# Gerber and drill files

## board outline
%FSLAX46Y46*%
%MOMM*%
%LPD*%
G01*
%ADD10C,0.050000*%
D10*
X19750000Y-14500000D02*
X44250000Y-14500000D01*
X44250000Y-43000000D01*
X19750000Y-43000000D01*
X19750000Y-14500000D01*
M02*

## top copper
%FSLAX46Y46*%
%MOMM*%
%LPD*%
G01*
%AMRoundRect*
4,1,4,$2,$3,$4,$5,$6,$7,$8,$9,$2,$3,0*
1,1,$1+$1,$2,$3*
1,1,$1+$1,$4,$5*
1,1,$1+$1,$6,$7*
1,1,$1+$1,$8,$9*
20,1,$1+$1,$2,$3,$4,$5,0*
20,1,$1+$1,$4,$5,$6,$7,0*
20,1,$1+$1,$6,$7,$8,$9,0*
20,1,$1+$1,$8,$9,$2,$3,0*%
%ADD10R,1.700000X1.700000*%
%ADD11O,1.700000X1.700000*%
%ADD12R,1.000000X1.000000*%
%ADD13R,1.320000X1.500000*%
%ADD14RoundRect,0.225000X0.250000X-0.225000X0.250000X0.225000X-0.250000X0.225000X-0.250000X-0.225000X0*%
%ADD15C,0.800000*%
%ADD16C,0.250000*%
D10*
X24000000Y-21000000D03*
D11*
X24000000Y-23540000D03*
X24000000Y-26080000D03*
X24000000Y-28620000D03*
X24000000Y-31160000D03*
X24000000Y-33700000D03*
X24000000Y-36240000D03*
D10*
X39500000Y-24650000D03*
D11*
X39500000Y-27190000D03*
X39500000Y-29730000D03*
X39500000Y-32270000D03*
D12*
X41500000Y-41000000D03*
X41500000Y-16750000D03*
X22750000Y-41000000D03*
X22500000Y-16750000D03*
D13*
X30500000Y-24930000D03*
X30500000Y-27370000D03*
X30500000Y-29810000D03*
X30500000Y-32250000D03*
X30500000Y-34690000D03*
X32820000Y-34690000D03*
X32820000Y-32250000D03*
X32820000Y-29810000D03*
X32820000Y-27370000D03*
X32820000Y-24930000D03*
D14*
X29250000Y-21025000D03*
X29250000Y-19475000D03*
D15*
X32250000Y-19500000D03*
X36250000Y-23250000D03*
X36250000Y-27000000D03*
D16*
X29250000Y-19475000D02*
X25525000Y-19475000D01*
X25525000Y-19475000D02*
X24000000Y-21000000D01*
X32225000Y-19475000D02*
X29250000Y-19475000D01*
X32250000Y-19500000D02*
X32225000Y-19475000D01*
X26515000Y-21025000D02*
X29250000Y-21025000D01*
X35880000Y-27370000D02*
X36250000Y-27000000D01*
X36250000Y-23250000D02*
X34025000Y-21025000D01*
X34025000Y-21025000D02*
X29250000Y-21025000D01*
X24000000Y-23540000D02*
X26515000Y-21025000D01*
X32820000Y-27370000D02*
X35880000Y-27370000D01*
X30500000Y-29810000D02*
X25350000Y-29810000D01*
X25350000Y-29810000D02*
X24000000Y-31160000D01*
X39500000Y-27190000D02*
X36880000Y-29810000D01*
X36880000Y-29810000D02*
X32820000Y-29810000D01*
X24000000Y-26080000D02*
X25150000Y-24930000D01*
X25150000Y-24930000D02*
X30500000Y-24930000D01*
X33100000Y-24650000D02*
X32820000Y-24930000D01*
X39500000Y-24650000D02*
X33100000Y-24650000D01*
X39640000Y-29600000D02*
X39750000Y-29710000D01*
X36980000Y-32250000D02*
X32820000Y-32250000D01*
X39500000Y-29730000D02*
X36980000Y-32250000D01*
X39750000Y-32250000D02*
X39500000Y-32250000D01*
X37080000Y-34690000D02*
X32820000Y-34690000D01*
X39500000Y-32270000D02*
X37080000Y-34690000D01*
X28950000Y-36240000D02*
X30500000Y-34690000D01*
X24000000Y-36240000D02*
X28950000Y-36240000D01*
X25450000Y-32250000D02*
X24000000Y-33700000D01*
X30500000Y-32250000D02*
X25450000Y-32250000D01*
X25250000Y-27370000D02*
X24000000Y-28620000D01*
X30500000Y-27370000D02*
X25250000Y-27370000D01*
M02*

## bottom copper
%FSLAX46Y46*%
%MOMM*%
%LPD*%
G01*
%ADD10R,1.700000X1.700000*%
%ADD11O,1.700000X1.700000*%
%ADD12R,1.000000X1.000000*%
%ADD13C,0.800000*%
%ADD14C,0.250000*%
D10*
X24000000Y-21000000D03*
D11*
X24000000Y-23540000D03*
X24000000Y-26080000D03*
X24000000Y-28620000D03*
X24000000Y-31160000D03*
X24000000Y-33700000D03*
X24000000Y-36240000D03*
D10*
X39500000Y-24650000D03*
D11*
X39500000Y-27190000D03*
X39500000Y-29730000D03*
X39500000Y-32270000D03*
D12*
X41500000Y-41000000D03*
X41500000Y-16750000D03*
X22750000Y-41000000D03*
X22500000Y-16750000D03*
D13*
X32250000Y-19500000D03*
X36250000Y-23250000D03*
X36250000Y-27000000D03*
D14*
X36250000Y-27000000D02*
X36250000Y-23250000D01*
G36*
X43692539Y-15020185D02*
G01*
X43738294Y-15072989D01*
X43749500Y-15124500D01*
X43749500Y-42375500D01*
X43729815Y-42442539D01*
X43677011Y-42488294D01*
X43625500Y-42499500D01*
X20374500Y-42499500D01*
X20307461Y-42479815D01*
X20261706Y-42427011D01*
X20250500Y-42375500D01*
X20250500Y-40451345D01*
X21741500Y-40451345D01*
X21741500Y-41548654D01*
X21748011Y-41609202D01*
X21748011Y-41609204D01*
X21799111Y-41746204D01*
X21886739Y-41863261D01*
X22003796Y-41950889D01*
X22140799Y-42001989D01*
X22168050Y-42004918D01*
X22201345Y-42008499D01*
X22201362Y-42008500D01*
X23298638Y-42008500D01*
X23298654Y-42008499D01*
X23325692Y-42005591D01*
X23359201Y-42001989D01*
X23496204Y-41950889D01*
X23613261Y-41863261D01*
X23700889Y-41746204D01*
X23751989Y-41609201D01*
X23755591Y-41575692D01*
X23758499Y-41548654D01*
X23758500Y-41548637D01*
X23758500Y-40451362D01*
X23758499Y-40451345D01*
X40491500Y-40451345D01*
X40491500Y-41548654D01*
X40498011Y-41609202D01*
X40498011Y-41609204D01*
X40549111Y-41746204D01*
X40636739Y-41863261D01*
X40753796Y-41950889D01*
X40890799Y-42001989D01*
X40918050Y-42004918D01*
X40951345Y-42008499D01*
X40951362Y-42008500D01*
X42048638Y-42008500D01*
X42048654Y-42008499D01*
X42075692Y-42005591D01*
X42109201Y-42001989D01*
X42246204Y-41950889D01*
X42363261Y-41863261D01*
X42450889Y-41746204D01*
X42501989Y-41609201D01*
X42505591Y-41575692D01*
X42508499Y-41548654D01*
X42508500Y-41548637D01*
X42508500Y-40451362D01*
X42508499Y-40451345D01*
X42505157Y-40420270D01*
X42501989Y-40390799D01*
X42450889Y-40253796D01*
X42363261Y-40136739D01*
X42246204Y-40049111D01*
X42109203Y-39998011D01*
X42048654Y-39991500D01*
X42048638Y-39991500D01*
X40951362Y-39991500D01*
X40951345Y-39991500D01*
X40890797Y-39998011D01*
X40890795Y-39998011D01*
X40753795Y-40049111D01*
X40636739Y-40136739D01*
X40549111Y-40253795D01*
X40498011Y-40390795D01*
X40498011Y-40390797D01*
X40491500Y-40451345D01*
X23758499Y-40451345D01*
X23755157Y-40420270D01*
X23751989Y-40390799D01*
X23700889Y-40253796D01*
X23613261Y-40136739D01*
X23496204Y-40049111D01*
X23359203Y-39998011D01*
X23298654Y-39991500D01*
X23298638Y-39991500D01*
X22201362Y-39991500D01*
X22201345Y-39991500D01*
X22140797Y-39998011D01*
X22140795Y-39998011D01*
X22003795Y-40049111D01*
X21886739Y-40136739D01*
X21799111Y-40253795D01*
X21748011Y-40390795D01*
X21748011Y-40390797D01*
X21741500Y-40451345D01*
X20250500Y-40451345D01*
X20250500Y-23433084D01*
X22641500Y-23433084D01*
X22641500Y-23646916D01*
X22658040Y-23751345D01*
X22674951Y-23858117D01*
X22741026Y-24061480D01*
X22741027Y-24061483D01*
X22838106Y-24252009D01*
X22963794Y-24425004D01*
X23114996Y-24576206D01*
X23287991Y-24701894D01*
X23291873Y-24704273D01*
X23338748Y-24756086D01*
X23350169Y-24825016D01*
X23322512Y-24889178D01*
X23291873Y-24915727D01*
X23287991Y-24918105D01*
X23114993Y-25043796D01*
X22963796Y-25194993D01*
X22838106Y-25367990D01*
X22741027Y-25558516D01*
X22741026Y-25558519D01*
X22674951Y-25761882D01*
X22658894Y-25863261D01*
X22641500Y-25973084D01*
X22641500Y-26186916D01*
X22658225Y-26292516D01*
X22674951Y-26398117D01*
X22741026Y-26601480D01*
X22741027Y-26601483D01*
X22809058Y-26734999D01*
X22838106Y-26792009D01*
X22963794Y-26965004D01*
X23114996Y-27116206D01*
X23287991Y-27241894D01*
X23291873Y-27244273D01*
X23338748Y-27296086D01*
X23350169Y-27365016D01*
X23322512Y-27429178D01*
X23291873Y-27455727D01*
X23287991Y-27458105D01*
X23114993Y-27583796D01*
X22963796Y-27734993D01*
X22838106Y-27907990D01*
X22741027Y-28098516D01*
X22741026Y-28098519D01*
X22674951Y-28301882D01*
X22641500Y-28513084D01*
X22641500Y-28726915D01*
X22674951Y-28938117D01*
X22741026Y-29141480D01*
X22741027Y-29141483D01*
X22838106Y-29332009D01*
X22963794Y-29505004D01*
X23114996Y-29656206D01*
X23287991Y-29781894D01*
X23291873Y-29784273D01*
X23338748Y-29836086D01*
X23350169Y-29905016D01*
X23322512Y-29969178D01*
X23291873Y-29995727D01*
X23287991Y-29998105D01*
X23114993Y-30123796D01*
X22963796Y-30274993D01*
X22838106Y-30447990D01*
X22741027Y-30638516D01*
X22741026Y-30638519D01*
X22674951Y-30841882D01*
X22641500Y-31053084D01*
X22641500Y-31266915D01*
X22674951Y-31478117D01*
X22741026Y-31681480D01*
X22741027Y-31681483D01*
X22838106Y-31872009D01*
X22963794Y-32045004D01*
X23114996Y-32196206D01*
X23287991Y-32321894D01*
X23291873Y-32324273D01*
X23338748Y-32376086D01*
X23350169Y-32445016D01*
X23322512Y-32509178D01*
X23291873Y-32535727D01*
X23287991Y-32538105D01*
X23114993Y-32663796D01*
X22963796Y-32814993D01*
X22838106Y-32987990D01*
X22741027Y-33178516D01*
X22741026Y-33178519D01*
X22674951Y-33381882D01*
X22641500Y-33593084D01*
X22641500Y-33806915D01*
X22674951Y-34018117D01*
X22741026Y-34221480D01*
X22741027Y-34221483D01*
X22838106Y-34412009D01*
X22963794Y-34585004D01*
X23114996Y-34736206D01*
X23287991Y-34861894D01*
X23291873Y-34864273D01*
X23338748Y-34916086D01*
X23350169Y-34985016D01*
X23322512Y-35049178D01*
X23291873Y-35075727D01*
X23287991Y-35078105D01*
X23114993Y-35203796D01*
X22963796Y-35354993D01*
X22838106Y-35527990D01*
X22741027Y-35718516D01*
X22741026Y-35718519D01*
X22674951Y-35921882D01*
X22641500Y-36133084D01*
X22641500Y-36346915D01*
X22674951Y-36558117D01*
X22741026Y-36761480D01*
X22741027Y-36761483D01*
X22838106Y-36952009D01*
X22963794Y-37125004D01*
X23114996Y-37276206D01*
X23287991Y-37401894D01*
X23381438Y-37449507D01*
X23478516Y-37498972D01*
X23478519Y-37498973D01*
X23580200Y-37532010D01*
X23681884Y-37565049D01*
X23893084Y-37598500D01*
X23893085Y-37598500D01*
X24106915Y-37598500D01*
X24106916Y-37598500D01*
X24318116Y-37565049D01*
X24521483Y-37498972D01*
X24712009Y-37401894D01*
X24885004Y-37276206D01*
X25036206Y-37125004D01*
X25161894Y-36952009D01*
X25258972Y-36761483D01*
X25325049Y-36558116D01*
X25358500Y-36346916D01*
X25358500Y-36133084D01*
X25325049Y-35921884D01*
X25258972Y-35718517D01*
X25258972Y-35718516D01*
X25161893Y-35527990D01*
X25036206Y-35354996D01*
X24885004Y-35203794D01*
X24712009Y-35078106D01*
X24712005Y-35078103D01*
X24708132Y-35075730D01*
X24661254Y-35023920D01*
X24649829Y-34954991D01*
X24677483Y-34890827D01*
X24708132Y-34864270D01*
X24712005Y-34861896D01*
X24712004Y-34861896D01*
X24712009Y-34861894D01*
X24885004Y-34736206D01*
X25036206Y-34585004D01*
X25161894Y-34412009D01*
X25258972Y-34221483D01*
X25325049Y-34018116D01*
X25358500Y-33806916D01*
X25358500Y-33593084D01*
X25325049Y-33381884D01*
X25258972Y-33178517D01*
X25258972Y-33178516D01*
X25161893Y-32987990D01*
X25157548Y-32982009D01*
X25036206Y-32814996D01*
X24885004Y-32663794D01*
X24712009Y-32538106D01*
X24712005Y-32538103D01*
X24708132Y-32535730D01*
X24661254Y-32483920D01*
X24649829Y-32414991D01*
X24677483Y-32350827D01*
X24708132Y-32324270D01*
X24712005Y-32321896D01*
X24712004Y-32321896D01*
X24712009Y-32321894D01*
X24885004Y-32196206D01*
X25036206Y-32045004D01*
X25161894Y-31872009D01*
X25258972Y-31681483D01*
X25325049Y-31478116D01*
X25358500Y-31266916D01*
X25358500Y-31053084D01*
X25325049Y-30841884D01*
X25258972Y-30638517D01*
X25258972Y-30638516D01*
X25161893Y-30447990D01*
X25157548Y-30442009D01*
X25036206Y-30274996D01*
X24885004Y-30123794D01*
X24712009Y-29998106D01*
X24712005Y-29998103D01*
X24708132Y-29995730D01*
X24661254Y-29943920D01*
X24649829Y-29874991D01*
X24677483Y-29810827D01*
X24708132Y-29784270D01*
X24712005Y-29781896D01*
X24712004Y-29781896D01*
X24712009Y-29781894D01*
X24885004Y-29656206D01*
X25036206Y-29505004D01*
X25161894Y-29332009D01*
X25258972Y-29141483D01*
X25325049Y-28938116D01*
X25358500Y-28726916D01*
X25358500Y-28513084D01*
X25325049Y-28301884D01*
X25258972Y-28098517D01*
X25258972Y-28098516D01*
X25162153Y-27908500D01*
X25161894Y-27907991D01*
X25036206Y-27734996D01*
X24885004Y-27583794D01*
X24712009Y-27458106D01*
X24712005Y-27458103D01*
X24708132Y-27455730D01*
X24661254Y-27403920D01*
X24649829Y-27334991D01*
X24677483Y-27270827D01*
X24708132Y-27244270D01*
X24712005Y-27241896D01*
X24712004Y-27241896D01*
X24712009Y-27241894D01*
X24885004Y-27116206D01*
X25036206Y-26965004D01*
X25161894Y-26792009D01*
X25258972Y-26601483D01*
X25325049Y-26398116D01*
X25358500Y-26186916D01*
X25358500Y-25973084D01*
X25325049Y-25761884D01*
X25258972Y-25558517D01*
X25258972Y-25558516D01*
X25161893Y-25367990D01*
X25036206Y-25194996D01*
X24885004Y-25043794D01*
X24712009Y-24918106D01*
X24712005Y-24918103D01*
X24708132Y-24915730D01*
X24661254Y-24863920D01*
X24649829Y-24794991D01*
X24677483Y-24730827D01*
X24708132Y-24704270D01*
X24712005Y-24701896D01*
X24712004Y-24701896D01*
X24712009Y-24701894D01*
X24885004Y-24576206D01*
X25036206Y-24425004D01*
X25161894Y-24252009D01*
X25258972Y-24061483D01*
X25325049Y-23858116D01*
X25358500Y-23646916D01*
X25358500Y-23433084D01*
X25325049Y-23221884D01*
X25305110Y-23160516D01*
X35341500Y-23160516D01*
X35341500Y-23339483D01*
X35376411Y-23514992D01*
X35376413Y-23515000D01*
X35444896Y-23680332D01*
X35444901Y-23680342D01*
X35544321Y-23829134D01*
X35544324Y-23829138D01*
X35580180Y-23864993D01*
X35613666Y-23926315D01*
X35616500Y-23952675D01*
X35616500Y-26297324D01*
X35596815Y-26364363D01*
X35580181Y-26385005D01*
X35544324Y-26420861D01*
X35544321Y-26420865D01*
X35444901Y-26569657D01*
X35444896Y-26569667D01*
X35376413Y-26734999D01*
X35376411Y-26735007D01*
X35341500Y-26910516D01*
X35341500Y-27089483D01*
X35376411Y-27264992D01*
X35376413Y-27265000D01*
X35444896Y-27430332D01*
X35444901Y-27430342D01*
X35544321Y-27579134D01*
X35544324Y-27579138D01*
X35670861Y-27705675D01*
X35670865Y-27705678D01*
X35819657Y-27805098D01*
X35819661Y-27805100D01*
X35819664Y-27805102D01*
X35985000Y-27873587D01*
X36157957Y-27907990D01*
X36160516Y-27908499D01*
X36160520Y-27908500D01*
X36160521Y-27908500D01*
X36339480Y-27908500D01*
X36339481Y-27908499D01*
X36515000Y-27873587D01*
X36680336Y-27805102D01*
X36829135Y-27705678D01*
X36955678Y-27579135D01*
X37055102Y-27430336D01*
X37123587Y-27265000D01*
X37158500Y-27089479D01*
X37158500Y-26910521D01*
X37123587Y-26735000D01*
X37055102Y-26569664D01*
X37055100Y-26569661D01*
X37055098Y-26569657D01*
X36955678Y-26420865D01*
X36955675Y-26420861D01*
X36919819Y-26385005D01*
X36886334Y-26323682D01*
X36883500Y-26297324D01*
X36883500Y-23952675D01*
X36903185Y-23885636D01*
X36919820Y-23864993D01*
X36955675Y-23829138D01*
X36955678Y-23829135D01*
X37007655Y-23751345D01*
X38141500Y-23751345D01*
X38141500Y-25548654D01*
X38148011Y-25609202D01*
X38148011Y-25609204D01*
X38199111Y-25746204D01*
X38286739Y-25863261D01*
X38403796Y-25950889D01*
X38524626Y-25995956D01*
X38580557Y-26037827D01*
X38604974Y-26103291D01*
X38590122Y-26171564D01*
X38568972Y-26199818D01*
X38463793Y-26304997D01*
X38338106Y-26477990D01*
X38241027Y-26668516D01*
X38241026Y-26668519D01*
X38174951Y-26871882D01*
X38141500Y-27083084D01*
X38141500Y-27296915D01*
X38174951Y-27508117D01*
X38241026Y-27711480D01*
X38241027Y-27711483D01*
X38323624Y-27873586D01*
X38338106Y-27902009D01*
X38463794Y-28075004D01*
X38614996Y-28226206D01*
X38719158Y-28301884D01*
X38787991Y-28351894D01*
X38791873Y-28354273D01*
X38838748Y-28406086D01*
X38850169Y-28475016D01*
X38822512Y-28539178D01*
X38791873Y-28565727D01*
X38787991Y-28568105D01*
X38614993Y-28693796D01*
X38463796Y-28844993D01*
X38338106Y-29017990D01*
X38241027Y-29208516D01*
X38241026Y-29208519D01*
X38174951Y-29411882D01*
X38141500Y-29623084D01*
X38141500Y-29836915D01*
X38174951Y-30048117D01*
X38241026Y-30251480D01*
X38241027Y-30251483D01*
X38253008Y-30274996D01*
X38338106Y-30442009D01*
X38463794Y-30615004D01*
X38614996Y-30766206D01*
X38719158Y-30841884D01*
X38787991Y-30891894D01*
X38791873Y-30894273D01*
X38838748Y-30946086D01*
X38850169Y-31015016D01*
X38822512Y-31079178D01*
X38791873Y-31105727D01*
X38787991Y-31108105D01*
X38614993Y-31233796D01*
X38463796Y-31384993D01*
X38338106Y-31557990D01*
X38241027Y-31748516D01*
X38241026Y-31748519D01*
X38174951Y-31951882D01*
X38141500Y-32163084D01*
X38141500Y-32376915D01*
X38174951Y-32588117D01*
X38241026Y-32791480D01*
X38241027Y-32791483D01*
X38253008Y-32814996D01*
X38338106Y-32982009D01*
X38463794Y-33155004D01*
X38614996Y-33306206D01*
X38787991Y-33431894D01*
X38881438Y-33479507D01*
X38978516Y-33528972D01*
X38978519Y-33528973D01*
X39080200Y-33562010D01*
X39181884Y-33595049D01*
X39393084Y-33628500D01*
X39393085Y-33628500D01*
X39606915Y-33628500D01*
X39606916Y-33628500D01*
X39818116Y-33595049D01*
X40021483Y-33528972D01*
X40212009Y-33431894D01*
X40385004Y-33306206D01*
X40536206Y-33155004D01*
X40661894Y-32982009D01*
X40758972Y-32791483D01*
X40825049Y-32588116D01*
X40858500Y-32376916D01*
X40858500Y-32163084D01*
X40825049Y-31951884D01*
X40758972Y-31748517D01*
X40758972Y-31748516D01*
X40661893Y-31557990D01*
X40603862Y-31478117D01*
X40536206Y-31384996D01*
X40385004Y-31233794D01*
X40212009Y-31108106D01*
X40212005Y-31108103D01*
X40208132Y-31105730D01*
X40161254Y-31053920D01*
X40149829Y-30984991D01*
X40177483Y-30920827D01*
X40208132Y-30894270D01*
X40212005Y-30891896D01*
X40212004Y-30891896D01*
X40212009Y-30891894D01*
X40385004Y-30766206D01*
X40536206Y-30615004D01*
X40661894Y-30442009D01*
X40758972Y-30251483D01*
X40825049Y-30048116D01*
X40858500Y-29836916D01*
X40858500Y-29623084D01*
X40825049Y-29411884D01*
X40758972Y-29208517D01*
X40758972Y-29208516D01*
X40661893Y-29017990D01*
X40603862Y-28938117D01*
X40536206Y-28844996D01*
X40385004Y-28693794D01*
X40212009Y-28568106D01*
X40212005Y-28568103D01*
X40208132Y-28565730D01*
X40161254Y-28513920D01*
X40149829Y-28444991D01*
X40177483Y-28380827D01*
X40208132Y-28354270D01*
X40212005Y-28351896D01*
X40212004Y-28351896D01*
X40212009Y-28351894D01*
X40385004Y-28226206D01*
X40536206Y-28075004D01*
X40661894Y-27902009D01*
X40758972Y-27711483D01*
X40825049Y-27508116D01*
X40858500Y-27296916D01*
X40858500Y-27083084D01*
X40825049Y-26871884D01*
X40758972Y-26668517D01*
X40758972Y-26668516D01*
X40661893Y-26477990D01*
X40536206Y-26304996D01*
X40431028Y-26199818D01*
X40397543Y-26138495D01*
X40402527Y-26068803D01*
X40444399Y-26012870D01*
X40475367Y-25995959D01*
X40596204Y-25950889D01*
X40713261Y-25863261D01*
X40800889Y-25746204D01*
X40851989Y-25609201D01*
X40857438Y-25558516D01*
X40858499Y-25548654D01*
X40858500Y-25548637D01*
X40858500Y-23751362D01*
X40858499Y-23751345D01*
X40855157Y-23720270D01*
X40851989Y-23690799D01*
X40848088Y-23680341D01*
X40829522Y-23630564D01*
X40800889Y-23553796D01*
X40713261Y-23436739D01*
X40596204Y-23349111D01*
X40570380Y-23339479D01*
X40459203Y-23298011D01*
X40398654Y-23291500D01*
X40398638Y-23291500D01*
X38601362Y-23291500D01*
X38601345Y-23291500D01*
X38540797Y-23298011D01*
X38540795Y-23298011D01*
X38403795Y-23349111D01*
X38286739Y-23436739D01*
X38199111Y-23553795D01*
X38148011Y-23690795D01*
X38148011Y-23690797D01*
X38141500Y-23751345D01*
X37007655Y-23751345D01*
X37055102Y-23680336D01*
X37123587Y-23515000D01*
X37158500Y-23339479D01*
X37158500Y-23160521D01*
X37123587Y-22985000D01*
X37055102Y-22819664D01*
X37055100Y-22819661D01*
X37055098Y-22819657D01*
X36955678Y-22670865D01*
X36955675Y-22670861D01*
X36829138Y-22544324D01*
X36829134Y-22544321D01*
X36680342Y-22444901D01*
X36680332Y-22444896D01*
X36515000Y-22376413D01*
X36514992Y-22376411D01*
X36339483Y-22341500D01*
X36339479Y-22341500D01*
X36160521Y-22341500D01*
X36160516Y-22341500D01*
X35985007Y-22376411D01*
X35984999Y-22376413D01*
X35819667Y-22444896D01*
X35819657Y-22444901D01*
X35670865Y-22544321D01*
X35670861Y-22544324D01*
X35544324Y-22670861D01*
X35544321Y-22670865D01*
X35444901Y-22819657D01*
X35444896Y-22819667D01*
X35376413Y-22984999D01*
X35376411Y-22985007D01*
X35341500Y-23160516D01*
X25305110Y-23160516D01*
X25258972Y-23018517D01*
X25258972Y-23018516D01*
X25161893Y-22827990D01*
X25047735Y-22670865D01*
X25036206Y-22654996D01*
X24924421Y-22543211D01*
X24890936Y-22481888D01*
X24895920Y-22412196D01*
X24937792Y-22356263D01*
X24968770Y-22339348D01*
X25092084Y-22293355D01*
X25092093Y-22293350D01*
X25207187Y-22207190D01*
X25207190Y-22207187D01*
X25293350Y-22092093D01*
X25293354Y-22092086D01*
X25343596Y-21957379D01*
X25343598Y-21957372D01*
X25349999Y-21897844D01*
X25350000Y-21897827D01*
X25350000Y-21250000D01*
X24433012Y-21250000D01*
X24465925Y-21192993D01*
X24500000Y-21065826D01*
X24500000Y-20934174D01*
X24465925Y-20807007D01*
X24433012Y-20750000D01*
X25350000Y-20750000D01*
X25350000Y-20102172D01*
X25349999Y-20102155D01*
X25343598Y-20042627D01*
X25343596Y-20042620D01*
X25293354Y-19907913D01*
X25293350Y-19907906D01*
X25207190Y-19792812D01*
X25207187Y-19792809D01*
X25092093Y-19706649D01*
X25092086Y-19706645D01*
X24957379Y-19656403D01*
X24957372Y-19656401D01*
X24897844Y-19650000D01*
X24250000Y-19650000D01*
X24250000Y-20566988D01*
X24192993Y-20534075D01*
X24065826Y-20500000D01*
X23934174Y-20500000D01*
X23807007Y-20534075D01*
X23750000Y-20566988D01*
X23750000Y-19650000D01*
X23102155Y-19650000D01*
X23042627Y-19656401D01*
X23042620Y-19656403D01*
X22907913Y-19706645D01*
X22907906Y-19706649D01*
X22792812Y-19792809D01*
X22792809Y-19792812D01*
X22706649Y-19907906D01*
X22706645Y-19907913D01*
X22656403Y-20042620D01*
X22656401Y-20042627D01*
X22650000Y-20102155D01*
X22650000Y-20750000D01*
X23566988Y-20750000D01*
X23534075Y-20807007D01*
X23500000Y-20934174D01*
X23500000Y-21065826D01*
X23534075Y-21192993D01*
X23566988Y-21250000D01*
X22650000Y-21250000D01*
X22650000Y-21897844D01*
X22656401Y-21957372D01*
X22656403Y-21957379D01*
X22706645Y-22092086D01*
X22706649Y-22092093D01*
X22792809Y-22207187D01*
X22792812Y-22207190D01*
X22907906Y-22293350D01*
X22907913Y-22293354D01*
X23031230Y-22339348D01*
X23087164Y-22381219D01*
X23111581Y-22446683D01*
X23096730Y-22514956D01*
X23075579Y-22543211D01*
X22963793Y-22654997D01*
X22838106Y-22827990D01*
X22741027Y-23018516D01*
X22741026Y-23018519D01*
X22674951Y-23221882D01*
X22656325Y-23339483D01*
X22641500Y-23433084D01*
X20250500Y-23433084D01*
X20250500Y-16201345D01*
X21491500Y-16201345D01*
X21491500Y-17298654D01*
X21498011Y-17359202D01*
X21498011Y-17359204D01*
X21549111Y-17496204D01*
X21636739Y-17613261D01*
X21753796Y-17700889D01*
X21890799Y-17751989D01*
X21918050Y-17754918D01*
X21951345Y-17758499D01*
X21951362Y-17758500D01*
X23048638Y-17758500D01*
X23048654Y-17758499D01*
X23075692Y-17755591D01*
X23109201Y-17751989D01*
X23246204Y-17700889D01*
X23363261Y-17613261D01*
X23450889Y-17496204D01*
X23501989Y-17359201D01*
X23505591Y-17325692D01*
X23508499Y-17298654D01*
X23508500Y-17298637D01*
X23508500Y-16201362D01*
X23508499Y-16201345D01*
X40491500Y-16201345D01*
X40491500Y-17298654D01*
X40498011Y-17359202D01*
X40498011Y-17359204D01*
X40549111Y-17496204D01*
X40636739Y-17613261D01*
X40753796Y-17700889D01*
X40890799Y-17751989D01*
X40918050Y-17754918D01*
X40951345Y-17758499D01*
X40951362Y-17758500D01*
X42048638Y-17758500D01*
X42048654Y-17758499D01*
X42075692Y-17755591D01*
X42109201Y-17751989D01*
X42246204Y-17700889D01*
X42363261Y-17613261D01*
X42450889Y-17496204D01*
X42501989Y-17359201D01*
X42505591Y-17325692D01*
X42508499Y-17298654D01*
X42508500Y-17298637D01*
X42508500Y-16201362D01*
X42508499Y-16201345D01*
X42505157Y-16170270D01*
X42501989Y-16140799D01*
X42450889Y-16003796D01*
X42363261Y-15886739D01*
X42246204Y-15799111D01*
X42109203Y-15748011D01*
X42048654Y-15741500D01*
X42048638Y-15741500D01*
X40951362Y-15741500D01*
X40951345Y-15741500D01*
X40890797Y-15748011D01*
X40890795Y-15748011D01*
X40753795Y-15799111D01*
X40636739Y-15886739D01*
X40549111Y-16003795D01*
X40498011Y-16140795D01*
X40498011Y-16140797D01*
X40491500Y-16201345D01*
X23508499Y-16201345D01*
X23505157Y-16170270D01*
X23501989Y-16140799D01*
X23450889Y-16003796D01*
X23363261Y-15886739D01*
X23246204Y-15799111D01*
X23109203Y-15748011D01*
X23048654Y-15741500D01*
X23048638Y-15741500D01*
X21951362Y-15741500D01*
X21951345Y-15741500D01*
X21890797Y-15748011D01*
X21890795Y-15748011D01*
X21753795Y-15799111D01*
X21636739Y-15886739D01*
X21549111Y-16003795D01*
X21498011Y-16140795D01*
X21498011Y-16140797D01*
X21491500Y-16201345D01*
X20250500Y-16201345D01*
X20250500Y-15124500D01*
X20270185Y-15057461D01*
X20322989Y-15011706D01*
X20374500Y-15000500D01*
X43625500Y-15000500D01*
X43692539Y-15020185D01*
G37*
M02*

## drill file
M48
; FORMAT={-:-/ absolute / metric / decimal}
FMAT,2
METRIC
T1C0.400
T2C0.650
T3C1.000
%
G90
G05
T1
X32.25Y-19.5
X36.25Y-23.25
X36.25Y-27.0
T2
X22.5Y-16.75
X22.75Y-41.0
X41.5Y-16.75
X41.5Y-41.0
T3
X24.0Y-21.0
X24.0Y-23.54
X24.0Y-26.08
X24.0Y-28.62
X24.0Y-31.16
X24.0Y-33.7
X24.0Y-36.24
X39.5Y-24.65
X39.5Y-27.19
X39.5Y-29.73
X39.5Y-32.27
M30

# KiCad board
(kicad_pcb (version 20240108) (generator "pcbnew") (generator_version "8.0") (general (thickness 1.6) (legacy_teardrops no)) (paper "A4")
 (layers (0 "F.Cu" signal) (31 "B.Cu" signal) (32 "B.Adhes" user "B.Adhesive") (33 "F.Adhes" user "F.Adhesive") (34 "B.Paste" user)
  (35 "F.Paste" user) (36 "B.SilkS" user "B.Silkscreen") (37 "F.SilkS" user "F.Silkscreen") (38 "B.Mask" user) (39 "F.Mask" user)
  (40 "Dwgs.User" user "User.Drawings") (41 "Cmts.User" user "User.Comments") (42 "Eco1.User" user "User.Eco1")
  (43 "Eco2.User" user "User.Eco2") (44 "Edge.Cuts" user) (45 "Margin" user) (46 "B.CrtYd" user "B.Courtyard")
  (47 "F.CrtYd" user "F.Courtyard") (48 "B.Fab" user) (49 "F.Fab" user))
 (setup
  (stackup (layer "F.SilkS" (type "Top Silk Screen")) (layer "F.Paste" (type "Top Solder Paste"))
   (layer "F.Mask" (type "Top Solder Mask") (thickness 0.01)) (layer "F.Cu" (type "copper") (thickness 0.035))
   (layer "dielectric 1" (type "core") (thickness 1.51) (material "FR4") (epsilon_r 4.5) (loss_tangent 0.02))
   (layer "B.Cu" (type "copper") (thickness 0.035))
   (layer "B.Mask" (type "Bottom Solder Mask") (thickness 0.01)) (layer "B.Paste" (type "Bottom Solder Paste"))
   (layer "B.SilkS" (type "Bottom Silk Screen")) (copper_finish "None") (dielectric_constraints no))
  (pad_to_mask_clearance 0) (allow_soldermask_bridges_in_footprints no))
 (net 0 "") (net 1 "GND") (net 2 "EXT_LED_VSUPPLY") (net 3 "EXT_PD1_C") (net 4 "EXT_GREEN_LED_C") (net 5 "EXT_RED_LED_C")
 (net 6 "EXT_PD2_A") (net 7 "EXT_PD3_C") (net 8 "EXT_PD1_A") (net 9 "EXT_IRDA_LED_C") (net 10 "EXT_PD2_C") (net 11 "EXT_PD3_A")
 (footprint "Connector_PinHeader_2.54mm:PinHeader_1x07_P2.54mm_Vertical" (layer "F.Cu") (at 24 21)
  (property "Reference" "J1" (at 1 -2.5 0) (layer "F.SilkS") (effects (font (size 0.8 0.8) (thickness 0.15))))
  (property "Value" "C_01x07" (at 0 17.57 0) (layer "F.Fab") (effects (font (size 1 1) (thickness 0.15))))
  (pad "1" thru_hole rect (at 0 0) (size 1.7 1.7) (drill 1) (layers "*.Cu" "*.Mask") (remove_unused_layers no) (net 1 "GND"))
  (pad "2" thru_hole oval (at 0 2.54) (size 1.7 1.7) (drill 1) (layers "*.Cu" "*.Mask") (remove_unused_layers no) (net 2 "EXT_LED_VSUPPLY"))
  (pad "3" thru_hole oval (at 0 5.08) (size 1.7 1.7) (drill 1) (layers "*.Cu" "*.Mask") (remove_unused_layers no) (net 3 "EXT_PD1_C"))
  (pad "4" thru_hole oval (at 0 7.62) (size 1.7 1.7) (drill 1) (layers "*.Cu" "*.Mask") (remove_unused_layers no) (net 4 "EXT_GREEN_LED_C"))
  (pad "5" thru_hole oval (at 0 10.16) (size 1.7 1.7) (drill 1) (layers "*.Cu" "*.Mask") (remove_unused_layers no) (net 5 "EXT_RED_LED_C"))
  (pad "6" thru_hole oval (at 0 12.7) (size 1.7 1.7) (drill 1) (layers "*.Cu" "*.Mask") (remove_unused_layers no) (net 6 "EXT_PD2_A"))
  (pad "7" thru_hole oval (at 0 15.24) (size 1.7 1.7) (drill 1) (layers "*.Cu" "*.Mask") (remove_unused_layers no) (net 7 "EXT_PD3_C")))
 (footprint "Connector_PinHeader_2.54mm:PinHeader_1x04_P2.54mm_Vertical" (layer "F.Cu") (at 39.5 24.65)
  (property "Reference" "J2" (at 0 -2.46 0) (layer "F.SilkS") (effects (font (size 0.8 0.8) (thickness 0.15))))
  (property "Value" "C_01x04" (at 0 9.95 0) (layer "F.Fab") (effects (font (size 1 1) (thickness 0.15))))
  (pad "1" thru_hole rect (at 0 0) (size 1.7 1.7) (drill 1) (layers "*.Cu" "*.Mask") (remove_unused_layers no) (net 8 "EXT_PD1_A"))
  (pad "2" thru_hole oval (at 0 2.54) (size 1.7 1.7) (drill 1) (layers "*.Cu" "*.Mask") (remove_unused_layers no) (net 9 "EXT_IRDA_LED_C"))
  (pad "3" thru_hole oval (at 0 5.08) (size 1.7 1.7) (drill 1) (layers "*.Cu" "*.Mask") (remove_unused_layers no) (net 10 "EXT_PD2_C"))
  (pad "4" thru_hole oval (at 0 7.62) (size 1.7 1.7) (drill 1) (layers "*.Cu" "*.Mask") (remove_unused_layers no) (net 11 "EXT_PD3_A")))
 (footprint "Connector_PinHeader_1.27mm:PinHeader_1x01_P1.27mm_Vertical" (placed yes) (layer "F.Cu") (at 41.5 41 180)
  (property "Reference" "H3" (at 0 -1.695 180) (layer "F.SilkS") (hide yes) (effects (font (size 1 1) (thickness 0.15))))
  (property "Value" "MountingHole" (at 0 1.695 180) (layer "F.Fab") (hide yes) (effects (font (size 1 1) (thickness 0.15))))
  (pad "1" thru_hole rect (at 0 0 180) (size 1 1) (drill 0.65) (layers "*.Cu" "*.Mask") (remove_unused_layers no)))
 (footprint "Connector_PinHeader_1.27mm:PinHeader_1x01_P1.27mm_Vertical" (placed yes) (layer "F.Cu") (at 41.5 16.75)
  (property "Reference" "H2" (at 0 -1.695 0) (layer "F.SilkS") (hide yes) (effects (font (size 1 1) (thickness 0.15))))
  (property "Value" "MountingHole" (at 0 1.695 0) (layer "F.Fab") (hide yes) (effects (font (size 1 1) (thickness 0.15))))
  (pad "1" thru_hole rect (at 0 0) (size 1 1) (drill 0.65) (layers "*.Cu" "*.Mask") (remove_unused_layers no)))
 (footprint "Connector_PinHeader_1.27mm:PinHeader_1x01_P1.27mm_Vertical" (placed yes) (layer "F.Cu") (at 22.75 41 180)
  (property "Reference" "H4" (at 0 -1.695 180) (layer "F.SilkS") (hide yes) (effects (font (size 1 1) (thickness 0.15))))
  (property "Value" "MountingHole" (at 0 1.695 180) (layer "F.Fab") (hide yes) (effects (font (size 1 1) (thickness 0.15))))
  (pad "1" thru_hole rect (at 0 0 180) (size 1 1) (drill 0.65) (layers "*.Cu" "*.Mask") (remove_unused_layers no)))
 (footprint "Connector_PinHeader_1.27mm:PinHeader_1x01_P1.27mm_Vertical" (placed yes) (layer "F.Cu") (at 22.5 16.75)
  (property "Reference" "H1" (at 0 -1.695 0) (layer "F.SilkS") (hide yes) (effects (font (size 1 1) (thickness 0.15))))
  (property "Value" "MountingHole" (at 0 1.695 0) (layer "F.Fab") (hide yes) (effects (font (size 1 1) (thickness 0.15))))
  (pad "1" thru_hole rect (at 0 0) (size 1 1) (drill 0.65) (layers "*.Cu" "*.Mask") (remove_unused_layers no)))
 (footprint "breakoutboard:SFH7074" (layer "F.Cu") (at 31.66 29.81 -90)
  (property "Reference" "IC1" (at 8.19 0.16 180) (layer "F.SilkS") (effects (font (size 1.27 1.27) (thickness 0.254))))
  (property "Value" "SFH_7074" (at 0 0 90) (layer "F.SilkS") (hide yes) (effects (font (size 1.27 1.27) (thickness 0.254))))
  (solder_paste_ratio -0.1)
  (pad "1" smd rect (at -4.88 1.16) (size 1.32 1.5) (layers "F.Cu" "F.Paste" "F.Mask") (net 3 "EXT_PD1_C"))
  (pad "2" smd rect (at -2.44 1.16) (size 1.32 1.5) (layers "F.Cu" "F.Paste" "F.Mask") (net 4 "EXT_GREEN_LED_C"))
  (pad "3" smd rect (at 0 1.16) (size 1.32 1.5) (layers "F.Cu" "F.Paste" "F.Mask") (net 5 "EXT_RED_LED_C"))
  (pad "4" smd rect (at 2.44 1.16) (size 1.32 1.5) (layers "F.Cu" "F.Paste" "F.Mask") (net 6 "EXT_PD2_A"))
  (pad "5" smd rect (at 4.88 1.16) (size 1.32 1.5) (layers "F.Cu" "F.Paste" "F.Mask") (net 7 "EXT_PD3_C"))
  (pad "6" smd rect (at 4.88 -1.16) (size 1.32 1.5) (layers "F.Cu" "F.Paste" "F.Mask") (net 11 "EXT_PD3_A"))
  (pad "7" smd rect (at 2.44 -1.16) (size 1.32 1.5) (layers "F.Cu" "F.Paste" "F.Mask") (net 10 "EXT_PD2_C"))
  (pad "8" smd rect (at 0 -1.16) (size 1.32 1.5) (layers "F.Cu" "F.Paste" "F.Mask") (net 9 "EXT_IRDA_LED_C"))
  (pad "9" smd rect (at -2.44 -1.16) (size 1.32 1.5) (layers "F.Cu" "F.Paste" "F.Mask") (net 2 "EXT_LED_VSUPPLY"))
  (pad "10" smd rect (at -4.88 -1.16) (size 1.32 1.5) (layers "F.Cu" "F.Paste" "F.Mask") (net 8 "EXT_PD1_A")))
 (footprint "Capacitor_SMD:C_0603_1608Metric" (layer "F.Cu") (at 29.25 20.25 90)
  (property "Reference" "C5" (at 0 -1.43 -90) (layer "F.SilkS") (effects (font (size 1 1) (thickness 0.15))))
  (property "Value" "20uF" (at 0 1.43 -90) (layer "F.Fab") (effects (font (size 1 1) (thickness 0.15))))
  (pad "1" smd roundrect (at -0.775 0 90) (size 0.9 0.95) (layers "F.Cu" "F.Paste" "F.Mask") (roundrect_rratio 0.25)
   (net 2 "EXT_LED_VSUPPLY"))
  (pad "2" smd roundrect (at 0.775 0 90) (size 0.9 0.95) (layers "F.Cu" "F.Paste" "F.Mask") (roundrect_rratio 0.25) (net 1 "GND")))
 (gr_rect (start 19.75 14.5) (end 44.25 43) (stroke (width 0.05) (type solid)) (fill none) (layer "Edge.Cuts"))
 (segment (start 29.25 19.475) (end 25.525 19.475) (width 0.25) (layer "F.Cu") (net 1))
 (segment (start 25.525 19.475) (end 24 21) (width 0.25) (layer "F.Cu") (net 1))
 (segment (start 32.225 19.475) (end 29.25 19.475) (width 0.25) (layer "F.Cu") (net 1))
 (segment (start 32.25 19.5) (end 32.225 19.475) (width 0.25) (layer "F.Cu") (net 1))
 (via (at 32.25 19.5) (size 0.8) (drill 0.4) (layers "F.Cu" "B.Cu") (free yes) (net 1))
 (segment (start 26.515 21.025) (end 29.25 21.025) (width 0.25) (layer "F.Cu") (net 2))
 (segment (start 35.88 27.37) (end 36.25 27) (width 0.25) (layer "F.Cu") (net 2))
 (segment (start 36.25 23.25) (end 34.025 21.025) (width 0.25) (layer "F.Cu") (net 2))
 (segment (start 34.025 21.025) (end 29.25 21.025) (width 0.25) (layer "F.Cu") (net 2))
 (segment (start 24 23.54) (end 26.515 21.025) (width 0.25) (layer "F.Cu") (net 2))
 (segment (start 32.82 27.37) (end 35.88 27.37) (width 0.25) (layer "F.Cu") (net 2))
 (via (at 36.25 23.25) (size 0.8) (drill 0.4) (layers "F.Cu" "B.Cu") (free yes) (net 2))
 (via (at 36.25 27) (size 0.8) (drill 0.4) (layers "F.Cu" "B.Cu") (free yes) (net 2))
 (segment (start 36.25 27) (end 36.25 23.25) (width 0.25) (layer "B.Cu") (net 2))
 (segment (start 30.5 29.81) (end 25.35 29.81) (width 0.25) (layer "F.Cu") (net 5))
 (segment (start 25.35 29.81) (end 24 31.16) (width 0.25) (layer "F.Cu") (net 5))
 (segment (start 39.5 27.19) (end 36.88 29.81) (width 0.25) (layer "F.Cu") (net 9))
 (segment (start 36.88 29.81) (end 32.82 29.81) (width 0.25) (layer "F.Cu") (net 9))
 (segment (start 24 26.08) (end 25.15 24.93) (width 0.25) (layer "F.Cu") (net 3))
 (segment (start 25.15 24.93) (end 30.5 24.93) (width 0.25) (layer "F.Cu") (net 3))
 (segment (start 33.1 24.65) (end 32.82 24.93) (width 0.25) (layer "F.Cu") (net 8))
 (segment (start 39.5 24.65) (end 33.1 24.65) (width 0.25) (layer "F.Cu") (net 8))
 (segment (start 39.64 29.6) (end 39.75 29.71) (width 0.25) (layer "F.Cu") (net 10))
 (segment (start 36.98 32.25) (end 32.82 32.25) (width 0.25) (layer "F.Cu") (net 10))
 (segment (start 39.5 29.73) (end 36.98 32.25) (width 0.25) (layer "F.Cu") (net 10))
 (segment (start 39.75 32.25) (end 39.5 32.25) (width 0.25) (layer "F.Cu") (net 11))
 (segment (start 37.08 34.69) (end 32.82 34.69) (width 0.25) (layer "F.Cu") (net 11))
 (segment (start 39.5 32.27) (end 37.08 34.69) (width 0.25) (layer "F.Cu") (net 11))
 (segment (start 28.95 36.24) (end 30.5 34.69) (width 0.25) (layer "F.Cu") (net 7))
 (segment (start 24 36.24) (end 28.95 36.24) (width 0.25) (layer "F.Cu") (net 7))
 (segment (start 25.45 32.25) (end 24 33.7) (width 0.25) (layer "F.Cu") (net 6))
 (segment (start 30.5 32.25) (end 25.45 32.25) (width 0.25) (layer "F.Cu") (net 6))
 (segment (start 25.25 27.37) (end 24 28.62) (width 0.25) (layer "F.Cu") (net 4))
 (segment (start 30.5 27.37) (end 25.25 27.37) (width 0.25) (layer "F.Cu") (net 4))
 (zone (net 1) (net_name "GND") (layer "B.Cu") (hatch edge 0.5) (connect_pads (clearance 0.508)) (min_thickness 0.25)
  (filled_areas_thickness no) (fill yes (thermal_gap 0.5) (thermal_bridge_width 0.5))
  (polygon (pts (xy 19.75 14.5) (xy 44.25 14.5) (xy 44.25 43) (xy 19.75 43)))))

